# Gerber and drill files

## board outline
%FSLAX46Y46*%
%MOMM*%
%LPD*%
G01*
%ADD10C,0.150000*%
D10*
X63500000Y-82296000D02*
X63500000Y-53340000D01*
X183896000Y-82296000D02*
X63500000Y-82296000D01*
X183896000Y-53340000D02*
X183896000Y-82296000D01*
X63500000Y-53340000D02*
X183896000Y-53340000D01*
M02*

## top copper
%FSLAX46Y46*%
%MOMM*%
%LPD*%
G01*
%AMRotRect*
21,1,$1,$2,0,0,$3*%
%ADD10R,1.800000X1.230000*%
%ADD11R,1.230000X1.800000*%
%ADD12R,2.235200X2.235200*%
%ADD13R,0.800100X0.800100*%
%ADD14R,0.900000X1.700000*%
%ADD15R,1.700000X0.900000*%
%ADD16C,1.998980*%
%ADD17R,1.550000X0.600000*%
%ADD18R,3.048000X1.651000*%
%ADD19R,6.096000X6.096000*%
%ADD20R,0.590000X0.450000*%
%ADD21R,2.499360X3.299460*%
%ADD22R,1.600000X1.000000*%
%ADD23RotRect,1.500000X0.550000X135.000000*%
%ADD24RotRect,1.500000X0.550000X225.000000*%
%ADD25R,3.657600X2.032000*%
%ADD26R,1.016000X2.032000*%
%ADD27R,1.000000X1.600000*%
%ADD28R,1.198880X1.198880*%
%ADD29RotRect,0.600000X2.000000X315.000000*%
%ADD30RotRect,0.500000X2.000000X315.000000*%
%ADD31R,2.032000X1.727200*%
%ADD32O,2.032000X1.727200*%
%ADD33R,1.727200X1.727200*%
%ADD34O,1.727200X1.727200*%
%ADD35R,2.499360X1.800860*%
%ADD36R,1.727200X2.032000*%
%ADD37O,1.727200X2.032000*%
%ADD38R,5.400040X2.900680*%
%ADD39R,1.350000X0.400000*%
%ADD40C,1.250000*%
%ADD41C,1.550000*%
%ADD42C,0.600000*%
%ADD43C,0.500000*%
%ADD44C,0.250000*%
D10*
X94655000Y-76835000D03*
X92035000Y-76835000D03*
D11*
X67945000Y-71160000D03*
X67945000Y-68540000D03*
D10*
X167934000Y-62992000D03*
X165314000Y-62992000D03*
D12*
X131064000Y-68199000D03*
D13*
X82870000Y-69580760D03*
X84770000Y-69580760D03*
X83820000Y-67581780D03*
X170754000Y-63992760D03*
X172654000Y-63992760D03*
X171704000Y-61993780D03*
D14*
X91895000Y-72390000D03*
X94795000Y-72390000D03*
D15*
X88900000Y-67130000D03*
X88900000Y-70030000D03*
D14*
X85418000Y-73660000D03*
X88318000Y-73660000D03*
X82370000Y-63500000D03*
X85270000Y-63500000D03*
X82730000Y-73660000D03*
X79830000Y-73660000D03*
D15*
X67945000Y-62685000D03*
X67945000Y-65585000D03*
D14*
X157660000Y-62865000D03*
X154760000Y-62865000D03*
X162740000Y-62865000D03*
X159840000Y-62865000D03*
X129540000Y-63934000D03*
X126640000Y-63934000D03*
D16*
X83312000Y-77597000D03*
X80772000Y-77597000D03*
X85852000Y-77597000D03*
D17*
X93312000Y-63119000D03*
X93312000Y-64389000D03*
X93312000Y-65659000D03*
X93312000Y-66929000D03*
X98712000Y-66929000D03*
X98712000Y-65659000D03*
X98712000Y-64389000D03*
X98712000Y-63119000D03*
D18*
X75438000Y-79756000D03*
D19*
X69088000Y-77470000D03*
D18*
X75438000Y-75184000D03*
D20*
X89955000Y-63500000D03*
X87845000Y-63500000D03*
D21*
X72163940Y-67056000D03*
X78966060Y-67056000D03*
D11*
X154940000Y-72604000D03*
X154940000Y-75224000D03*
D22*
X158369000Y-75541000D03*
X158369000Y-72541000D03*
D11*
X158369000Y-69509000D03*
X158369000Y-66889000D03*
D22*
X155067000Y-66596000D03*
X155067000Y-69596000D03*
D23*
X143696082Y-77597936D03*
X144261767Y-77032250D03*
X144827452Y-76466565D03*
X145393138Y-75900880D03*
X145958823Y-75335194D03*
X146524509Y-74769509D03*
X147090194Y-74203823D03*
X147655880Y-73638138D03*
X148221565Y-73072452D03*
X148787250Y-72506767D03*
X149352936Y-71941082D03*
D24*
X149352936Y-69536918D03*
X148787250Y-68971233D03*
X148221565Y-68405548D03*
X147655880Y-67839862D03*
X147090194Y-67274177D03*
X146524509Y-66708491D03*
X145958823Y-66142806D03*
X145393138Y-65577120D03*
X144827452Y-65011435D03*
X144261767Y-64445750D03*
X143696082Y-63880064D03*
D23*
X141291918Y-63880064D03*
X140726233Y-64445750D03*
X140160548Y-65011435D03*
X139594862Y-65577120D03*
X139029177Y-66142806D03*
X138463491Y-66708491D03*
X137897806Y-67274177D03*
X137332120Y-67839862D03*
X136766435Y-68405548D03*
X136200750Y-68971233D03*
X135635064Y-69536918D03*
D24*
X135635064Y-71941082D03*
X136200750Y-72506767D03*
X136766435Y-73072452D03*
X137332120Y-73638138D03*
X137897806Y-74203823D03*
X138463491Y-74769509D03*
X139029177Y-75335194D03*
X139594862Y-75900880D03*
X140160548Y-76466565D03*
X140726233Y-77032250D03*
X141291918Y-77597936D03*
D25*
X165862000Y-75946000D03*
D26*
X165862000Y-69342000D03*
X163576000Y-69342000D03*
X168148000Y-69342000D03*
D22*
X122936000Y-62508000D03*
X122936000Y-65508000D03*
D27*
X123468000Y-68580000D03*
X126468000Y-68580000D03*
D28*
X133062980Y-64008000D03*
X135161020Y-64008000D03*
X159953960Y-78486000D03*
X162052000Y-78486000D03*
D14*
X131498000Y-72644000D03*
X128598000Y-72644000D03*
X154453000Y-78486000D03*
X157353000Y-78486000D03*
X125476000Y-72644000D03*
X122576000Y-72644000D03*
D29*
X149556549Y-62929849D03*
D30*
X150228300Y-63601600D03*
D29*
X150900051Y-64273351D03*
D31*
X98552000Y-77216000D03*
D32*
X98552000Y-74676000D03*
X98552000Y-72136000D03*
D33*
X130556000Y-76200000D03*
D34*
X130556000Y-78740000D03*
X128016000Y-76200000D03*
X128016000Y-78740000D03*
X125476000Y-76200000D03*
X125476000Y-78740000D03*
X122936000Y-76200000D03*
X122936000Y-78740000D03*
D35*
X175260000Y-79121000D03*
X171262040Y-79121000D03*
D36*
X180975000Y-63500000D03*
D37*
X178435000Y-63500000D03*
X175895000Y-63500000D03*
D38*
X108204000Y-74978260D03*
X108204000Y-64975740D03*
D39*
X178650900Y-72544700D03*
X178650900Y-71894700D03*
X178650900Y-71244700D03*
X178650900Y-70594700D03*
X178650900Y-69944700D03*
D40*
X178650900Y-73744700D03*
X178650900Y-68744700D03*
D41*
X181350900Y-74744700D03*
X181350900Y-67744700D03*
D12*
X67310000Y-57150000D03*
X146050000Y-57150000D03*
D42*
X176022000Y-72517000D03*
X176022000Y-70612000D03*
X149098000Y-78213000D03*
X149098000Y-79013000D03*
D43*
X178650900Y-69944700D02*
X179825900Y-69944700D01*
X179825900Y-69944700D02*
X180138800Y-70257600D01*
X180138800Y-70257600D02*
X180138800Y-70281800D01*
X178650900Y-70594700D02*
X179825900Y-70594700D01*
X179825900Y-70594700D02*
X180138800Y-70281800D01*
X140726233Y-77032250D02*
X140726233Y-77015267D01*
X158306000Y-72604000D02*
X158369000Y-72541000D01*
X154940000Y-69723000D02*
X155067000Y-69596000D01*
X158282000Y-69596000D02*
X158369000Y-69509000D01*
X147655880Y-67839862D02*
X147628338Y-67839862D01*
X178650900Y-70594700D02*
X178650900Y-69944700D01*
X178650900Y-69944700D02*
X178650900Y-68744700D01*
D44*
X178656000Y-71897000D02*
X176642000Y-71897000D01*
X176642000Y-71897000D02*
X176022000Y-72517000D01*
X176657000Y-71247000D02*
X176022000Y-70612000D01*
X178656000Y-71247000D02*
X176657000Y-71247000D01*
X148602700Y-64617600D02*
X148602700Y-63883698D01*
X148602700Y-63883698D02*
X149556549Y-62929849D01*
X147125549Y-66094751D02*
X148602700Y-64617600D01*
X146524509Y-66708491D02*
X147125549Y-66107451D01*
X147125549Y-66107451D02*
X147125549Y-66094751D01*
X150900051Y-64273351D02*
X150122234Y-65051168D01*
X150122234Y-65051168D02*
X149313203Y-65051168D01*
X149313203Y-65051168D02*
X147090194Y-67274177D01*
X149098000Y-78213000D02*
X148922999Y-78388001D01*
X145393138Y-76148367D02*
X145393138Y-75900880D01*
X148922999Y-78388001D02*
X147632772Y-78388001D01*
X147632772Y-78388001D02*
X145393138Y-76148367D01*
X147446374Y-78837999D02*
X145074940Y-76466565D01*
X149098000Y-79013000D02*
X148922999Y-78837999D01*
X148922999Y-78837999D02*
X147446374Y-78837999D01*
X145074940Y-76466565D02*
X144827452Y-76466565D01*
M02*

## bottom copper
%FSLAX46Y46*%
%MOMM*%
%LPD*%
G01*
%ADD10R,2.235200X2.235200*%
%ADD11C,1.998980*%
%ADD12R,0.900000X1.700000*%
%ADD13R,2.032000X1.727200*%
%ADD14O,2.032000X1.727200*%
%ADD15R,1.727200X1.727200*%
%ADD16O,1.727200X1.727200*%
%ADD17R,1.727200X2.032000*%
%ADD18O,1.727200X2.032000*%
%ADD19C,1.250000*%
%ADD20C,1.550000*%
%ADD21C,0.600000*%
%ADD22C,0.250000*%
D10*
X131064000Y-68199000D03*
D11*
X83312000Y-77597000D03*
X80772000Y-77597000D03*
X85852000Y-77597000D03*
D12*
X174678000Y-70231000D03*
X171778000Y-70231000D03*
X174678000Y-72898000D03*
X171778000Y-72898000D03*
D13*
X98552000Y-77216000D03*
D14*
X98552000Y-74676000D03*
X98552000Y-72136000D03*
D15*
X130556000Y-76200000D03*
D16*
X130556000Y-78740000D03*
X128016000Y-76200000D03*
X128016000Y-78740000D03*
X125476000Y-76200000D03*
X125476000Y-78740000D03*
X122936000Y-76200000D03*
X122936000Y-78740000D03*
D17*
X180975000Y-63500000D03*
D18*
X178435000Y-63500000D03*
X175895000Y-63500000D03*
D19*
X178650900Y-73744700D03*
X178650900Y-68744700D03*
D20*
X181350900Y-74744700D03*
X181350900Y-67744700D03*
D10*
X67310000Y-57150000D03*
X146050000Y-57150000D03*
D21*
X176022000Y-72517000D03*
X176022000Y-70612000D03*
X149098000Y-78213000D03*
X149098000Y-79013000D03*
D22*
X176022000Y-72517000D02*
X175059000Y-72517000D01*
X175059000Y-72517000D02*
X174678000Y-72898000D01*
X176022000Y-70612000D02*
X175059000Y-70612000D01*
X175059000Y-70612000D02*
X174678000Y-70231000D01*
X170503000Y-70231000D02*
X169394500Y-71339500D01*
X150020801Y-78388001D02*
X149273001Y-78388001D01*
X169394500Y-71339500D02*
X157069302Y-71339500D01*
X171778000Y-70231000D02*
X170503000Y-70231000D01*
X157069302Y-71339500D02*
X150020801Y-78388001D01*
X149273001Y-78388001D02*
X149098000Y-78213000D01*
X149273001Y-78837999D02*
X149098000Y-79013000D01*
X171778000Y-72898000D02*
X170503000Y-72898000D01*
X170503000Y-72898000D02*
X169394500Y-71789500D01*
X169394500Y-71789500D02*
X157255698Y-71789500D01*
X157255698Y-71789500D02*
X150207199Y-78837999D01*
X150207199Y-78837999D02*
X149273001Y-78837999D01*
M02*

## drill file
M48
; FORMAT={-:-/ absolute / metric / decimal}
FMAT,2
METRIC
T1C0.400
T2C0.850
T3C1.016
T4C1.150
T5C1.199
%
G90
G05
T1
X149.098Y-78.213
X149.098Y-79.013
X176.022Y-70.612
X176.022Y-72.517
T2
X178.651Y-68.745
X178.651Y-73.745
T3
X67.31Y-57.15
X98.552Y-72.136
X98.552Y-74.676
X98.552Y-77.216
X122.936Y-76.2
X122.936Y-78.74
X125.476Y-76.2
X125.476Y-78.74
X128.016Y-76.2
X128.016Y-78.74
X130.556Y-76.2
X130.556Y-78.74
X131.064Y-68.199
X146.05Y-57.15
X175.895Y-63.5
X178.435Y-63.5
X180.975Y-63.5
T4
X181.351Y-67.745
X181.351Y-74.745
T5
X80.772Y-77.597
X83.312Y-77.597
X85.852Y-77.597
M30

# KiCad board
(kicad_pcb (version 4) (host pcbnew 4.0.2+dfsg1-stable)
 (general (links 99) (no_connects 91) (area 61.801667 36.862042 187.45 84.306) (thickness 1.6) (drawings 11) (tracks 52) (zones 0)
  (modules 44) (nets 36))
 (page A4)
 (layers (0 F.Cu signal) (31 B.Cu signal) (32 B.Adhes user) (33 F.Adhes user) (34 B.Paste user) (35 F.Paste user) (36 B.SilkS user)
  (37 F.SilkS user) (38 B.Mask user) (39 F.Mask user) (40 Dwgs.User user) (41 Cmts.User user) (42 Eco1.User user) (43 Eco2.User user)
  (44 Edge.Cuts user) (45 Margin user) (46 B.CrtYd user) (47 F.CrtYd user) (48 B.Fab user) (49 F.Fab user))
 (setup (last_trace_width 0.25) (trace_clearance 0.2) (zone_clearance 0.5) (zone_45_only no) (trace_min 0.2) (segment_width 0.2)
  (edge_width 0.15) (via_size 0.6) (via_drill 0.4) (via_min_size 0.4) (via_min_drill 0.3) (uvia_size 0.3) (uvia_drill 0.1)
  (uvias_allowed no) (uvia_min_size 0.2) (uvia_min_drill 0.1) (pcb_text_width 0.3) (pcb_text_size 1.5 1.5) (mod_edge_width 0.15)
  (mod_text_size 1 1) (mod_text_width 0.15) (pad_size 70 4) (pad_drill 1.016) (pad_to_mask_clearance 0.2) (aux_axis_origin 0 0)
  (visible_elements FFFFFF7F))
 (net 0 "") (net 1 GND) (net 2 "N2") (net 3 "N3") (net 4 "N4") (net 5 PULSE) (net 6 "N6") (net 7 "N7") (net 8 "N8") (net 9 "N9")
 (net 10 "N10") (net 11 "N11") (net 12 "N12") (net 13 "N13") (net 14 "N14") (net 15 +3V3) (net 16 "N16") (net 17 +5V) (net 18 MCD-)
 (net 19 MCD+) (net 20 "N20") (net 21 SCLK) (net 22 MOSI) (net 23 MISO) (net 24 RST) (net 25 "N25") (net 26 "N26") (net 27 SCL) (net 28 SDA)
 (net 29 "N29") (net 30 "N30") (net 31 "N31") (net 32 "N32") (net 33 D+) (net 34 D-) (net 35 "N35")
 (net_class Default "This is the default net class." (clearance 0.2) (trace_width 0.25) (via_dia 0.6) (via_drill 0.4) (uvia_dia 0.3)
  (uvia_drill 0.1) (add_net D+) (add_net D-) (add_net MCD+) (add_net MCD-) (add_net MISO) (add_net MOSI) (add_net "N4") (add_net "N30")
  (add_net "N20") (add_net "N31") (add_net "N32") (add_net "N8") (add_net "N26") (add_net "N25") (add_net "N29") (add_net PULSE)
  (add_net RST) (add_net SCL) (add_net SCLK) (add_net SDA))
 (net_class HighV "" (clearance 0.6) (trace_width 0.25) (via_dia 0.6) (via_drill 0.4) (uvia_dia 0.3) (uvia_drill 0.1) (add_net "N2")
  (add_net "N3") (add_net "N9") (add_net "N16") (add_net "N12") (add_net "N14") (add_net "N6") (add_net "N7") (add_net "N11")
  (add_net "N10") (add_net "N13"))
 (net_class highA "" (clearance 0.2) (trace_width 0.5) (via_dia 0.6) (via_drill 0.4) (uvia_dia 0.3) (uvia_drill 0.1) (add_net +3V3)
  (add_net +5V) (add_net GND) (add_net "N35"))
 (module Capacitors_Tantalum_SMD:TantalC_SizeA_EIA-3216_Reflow (layer F.Cu) (at 93.345 76.835)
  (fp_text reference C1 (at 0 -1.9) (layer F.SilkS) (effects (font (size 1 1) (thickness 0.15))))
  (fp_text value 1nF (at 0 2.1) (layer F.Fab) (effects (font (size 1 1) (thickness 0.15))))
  (pad 2 smd rect (at 1.31 0) (size 1.8 1.23) (layers F.Cu F.Paste F.Mask) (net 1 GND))
  (pad 1 smd rect (at -1.31 0) (size 1.8 1.23) (layers F.Cu F.Paste F.Mask) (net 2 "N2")))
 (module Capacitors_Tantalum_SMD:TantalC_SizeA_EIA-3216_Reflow (layer F.Cu) (at 67.945 69.85 270)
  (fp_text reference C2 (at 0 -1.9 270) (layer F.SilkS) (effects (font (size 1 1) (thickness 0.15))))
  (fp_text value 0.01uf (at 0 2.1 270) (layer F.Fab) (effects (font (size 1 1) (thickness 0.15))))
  (pad 2 smd rect (at 1.31 0 270) (size 1.8 1.23) (layers F.Cu F.Paste F.Mask) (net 1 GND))
  (pad 1 smd rect (at -1.31 0 270) (size 1.8 1.23) (layers F.Cu F.Paste F.Mask) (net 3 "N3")))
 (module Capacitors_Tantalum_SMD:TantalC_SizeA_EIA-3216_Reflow (layer F.Cu) (at 166.624 62.992)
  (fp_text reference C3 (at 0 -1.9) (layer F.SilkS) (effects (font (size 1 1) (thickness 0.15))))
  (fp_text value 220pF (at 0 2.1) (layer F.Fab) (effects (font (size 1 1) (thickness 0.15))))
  (pad 2 smd rect (at 1.31 0) (size 1.8 1.23) (layers F.Cu F.Paste F.Mask) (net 1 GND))
  (pad 1 smd rect (at -1.31 0) (size 1.8 1.23) (layers F.Cu F.Paste F.Mask) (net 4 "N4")))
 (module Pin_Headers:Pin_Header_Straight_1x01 (layer F.Cu) (at 131.064 68.199)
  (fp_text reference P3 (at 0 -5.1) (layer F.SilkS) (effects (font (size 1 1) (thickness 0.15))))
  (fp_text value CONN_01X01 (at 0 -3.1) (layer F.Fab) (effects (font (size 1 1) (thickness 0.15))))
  (pad 1 thru_hole rect (at 0 0) (size 2.2352 2.2352) (drill 1.016) (layers *.Cu *.Mask F.SilkS) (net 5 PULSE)))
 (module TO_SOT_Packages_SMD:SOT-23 (layer F.Cu) (at 83.82 68.58)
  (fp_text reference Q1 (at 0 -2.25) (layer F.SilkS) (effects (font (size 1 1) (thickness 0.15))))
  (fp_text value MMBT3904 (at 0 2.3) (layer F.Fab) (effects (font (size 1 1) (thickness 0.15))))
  (pad 1 smd rect (at -0.95 1.00076) (size 0.8001 0.8001) (layers F.Cu F.Paste F.Mask) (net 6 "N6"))
  (pad 2 smd rect (at 0.95 1.00076) (size 0.8001 0.8001) (layers F.Cu F.Paste F.Mask) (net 1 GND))
  (pad 3 smd rect (at 0 -0.99822) (size 0.8001 0.8001) (layers F.Cu F.Paste F.Mask) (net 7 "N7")))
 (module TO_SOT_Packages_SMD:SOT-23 (layer F.Cu) (at 171.704 62.992)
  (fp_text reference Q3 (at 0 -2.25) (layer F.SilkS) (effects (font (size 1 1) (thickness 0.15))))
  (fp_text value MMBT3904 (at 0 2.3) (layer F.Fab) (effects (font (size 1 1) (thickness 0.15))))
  (pad 1 smd rect (at -0.95 1.00076) (size 0.8001 0.8001) (layers F.Cu F.Paste F.Mask) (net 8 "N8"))
  (pad 2 smd rect (at 0.95 1.00076) (size 0.8001 0.8001) (layers F.Cu F.Paste F.Mask) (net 1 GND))
  (pad 3 smd rect (at 0 -0.99822) (size 0.8001 0.8001) (layers F.Cu F.Paste F.Mask) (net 5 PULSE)))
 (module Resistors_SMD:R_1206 (layer F.Cu) (at 93.345 72.39)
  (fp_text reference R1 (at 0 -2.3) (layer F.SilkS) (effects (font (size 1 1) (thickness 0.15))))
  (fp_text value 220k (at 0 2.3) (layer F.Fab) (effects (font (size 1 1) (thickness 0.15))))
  (pad 1 smd rect (at -1.45 0) (size 0.9 1.7) (layers F.Cu F.Paste F.Mask) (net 2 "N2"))
  (pad 2 smd rect (at 1.45 0) (size 0.9 1.7) (layers F.Cu F.Paste F.Mask) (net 1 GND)))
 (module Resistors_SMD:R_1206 (layer F.Cu) (at 88.9 68.58 270)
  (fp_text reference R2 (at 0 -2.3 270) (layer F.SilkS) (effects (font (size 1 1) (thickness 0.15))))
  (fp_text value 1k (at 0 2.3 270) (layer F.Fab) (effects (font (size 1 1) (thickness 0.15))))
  (pad 1 smd rect (at -1.45 0 270) (size 0.9 1.7) (layers F.Cu F.Paste F.Mask) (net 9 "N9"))
  (pad 2 smd rect (at 1.45 0 270) (size 0.9 1.7) (layers F.Cu F.Paste F.Mask) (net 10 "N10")))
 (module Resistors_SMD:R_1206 (layer F.Cu) (at 86.868 73.66)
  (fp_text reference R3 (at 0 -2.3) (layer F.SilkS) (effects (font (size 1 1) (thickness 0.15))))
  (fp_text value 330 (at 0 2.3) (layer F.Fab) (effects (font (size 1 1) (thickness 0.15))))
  (pad 1 smd rect (at -1.45 0) (size 0.9 1.7) (layers F.Cu F.Paste F.Mask) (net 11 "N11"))
  (pad 2 smd rect (at 1.45 0) (size 0.9 1.7) (layers F.Cu F.Paste F.Mask) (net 10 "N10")))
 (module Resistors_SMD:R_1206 (layer F.Cu) (at 83.82 63.5)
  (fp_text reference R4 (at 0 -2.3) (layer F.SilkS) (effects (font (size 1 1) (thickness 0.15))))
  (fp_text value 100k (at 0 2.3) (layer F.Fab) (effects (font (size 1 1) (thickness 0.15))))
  (pad 1 smd rect (at -1.45 0) (size 0.9 1.7) (layers F.Cu F.Paste F.Mask) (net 7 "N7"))
  (pad 2 smd rect (at 1.45 0) (size 0.9 1.7) (layers F.Cu F.Paste F.Mask) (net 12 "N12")))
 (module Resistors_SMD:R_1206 (layer F.Cu) (at 81.28 73.66 180)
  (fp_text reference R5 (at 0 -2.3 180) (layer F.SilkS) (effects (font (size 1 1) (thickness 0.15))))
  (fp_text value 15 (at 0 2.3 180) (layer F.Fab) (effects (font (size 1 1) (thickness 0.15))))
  (pad 1 smd rect (at -1.45 0 180) (size 0.9 1.7) (layers F.Cu F.Paste F.Mask) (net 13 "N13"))
  (pad 2 smd rect (at 1.45 0 180) (size 0.9 1.7) (layers F.Cu F.Paste F.Mask) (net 6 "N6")))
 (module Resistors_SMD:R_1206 (layer F.Cu) (at 67.945 64.135 270)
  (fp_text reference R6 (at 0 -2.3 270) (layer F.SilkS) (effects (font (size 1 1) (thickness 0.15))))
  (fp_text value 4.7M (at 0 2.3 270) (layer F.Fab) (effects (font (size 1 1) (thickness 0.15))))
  (pad 1 smd rect (at -1.45 0 270) (size 0.9 1.7) (layers F.Cu F.Paste F.Mask) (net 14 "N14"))
  (pad 2 smd rect (at 1.45 0 270) (size 0.9 1.7) (layers F.Cu F.Paste F.Mask) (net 3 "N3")))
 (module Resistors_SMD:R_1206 (layer F.Cu) (at 156.21 62.865 180)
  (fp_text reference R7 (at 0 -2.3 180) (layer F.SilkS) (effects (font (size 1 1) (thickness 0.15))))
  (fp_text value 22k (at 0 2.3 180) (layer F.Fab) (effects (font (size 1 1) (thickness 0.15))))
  (pad 1 smd rect (at -1.45 0 180) (size 0.9 1.7) (layers F.Cu F.Paste F.Mask) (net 8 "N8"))
  (pad 2 smd rect (at 1.45 0 180) (size 0.9 1.7) (layers F.Cu F.Paste F.Mask) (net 4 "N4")))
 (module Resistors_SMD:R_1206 (layer F.Cu) (at 161.29 62.865 180)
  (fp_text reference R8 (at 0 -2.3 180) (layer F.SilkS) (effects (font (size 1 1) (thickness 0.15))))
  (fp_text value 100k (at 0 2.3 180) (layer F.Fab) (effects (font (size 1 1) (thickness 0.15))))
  (pad 1 smd rect (at -1.45 0 180) (size 0.9 1.7) (layers F.Cu F.Paste F.Mask) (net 1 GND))
  (pad 2 smd rect (at 1.45 0 180) (size 0.9 1.7) (layers F.Cu F.Paste F.Mask) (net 8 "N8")))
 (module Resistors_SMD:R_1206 (layer F.Cu) (at 128.09 63.934 180)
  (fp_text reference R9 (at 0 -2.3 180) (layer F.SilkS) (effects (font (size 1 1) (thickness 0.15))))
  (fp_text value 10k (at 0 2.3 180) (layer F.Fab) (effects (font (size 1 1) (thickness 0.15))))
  (pad 1 smd rect (at -1.45 0 180) (size 0.9 1.7) (layers F.Cu F.Paste F.Mask) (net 5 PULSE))
  (pad 2 smd rect (at 1.45 0 180) (size 0.9 1.7) (layers F.Cu F.Paste F.Mask) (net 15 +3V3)))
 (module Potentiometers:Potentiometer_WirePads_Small (layer F.Cu) (at 85.852 77.597 270)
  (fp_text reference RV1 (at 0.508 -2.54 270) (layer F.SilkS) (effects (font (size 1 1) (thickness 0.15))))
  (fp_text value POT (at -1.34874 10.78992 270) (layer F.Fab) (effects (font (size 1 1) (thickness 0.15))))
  (pad 2 thru_hole circle (at 0 2.54 270) (size 1.99898 1.99898) (drill 1.19888) (layers *.Cu *.Mask F.SilkS) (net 13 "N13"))
  (pad 3 thru_hole circle (at 0 5.08 270) (size 1.99898 1.99898) (drill 1.19888) (layers *.Cu *.Mask F.SilkS) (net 1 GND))
  (pad 1 thru_hole circle (at 0 0 270) (size 1.99898 1.99898) (drill 1.19888) (layers *.Cu *.Mask F.SilkS) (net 13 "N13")))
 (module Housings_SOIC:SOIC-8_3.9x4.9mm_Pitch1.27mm (layer F.Cu) (at 96.012 65.024)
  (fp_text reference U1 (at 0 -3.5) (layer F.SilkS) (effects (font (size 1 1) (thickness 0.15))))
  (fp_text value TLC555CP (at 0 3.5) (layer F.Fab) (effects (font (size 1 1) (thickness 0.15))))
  (pad 1 smd rect (at -2.7 -1.905) (size 1.55 0.6) (layers F.Cu F.Paste F.Mask) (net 1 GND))
  (pad 2 smd rect (at -2.7 -0.635) (size 1.55 0.6) (layers F.Cu F.Paste F.Mask) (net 2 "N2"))
  (pad 3 smd rect (at -2.7 0.635) (size 1.55 0.6) (layers F.Cu F.Paste F.Mask) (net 10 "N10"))
  (pad 4 smd rect (at -2.7 1.905) (size 1.55 0.6) (layers F.Cu F.Paste F.Mask) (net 7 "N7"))
  (pad 5 smd rect (at 2.7 1.905) (size 1.55 0.6) (layers F.Cu F.Paste F.Mask))
  (pad 6 smd rect (at 2.7 0.635) (size 1.55 0.6) (layers F.Cu F.Paste F.Mask) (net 1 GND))
  (pad 7 smd rect (at 2.7 -0.635) (size 1.55 0.6) (layers F.Cu F.Paste F.Mask) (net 11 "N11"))
  (pad 8 smd rect (at 2.7 -1.905) (size 1.55 0.6) (layers F.Cu F.Paste F.Mask) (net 12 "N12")))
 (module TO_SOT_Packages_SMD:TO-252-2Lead (layer F.Cu) (at 75.438 77.47 90)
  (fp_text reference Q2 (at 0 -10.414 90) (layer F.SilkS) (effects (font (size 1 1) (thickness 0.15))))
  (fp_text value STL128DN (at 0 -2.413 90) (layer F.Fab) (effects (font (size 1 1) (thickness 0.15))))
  (pad 1 smd rect (at -2.286 0 90) (size 1.651 3.048) (layers F.Cu F.Paste F.Mask) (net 11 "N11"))
  (pad 2 smd rect (at 0 -6.35 90) (size 6.096 6.096) (layers F.Cu F.Paste F.Mask) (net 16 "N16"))
  (pad 3 smd rect (at 2.286 0 90) (size 1.651 3.048) (layers F.Cu F.Paste F.Mask) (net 6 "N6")))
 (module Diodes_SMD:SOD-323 (layer F.Cu) (at 88.9 63.5 180)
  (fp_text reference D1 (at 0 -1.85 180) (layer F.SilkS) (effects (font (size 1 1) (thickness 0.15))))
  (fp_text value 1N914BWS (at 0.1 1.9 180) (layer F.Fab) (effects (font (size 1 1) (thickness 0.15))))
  (pad 1 smd rect (at -1.055 0 180) (size 0.59 0.45) (layers F.Cu F.Paste F.Mask) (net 2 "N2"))
  (pad 2 smd rect (at 1.055 0 180) (size 0.59 0.45) (layers F.Cu F.Paste F.Mask) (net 9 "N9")))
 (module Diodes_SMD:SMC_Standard (layer F.Cu) (at 75.565 67.056)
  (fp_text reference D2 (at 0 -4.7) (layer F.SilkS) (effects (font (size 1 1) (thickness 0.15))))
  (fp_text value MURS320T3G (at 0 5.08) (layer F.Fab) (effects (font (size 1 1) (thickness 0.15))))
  (pad 1 smd rect (at -3.40106 0 90) (size 3.29946 2.49936) (layers F.Cu F.Paste F.Mask) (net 3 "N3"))
  (pad 2 smd rect (at 3.40106 0 90) (size 3.29946 2.49936) (layers F.Cu F.Paste F.Mask) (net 16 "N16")))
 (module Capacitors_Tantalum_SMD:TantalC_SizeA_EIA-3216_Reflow (layer F.Cu) (at 154.94 73.914 90)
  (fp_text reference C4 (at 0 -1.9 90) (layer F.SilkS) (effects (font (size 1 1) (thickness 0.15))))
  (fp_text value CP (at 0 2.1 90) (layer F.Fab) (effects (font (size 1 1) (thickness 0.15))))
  (pad 2 smd rect (at 1.31 0 90) (size 1.8 1.23) (layers F.Cu F.Paste F.Mask) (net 1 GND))
  (pad 1 smd rect (at -1.31 0 90) (size 1.8 1.23) (layers F.Cu F.Paste F.Mask) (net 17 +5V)))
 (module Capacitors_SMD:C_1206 (layer F.Cu) (at 158.369 74.041 90)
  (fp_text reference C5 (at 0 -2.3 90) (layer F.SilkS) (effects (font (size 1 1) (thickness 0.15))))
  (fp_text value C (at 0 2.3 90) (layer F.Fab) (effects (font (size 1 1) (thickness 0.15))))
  (pad 1 smd rect (at -1.5 0 90) (size 1 1.6) (layers F.Cu F.Paste F.Mask) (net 17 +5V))
  (pad 2 smd rect (at 1.5 0 90) (size 1 1.6) (layers F.Cu F.Paste F.Mask) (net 1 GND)))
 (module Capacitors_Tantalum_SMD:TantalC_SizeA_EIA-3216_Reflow (layer F.Cu) (at 158.369 68.199 270)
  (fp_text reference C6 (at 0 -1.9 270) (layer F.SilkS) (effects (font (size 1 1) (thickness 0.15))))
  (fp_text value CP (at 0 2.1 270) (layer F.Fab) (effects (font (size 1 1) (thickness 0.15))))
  (pad 2 smd rect (at 1.31 0 270) (size 1.8 1.23) (layers F.Cu F.Paste F.Mask) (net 1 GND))
  (pad 1 smd rect (at -1.31 0 270) (size 1.8 1.23) (layers F.Cu F.Paste F.Mask) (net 15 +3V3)))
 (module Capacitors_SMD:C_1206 (layer F.Cu) (at 155.067 68.096 270)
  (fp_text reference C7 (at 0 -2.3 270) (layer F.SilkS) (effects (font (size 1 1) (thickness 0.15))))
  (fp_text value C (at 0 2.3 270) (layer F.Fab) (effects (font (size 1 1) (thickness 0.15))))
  (pad 1 smd rect (at -1.5 0 270) (size 1 1.6) (layers F.Cu F.Paste F.Mask) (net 15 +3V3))
  (pad 2 smd rect (at 1.5 0 270) (size 1 1.6) (layers F.Cu F.Paste F.Mask) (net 1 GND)))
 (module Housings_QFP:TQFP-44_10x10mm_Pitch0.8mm (layer F.Cu) (at 142.494 70.739 135)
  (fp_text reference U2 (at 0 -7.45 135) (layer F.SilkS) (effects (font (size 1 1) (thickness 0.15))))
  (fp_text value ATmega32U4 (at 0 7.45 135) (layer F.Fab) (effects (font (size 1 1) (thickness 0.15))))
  (pad 1 smd rect (at -5.7 -4 135) (size 1.5 0.55) (layers F.Cu F.Paste F.Mask))
  (pad 2 smd rect (at -5.7 -3.2 135) (size 1.5 0.55) (layers F.Cu F.Paste F.Mask) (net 17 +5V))
  (pad 3 smd rect (at -5.7 -2.4 135) (size 1.5 0.55) (layers F.Cu F.Paste F.Mask) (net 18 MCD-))
  (pad 4 smd rect (at -5.7 -1.6 135) (size 1.5 0.55) (layers F.Cu F.Paste F.Mask) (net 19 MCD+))
  (pad 5 smd rect (at -5.7 -0.8 135) (size 1.5 0.55) (layers F.Cu F.Paste F.Mask) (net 1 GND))
  (pad 6 smd rect (at -5.7 0 135) (size 1.5 0.55) (layers F.Cu F.Paste F.Mask) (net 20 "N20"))
  (pad 7 smd rect (at -5.7 0.8 135) (size 1.5 0.55) (layers F.Cu F.Paste F.Mask) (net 17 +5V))
  (pad 8 smd rect (at -5.7 1.6 135) (size 1.5 0.55) (layers F.Cu F.Paste F.Mask))
  (pad 9 smd rect (at -5.7 2.4 135) (size 1.5 0.55) (layers F.Cu F.Paste F.Mask) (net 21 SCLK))
  (pad 10 smd rect (at -5.7 3.2 135) (size 1.5 0.55) (layers F.Cu F.Paste F.Mask) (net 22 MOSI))
  (pad 11 smd rect (at -5.7 4 135) (size 1.5 0.55) (layers F.Cu F.Paste F.Mask) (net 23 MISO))
  (pad 12 smd rect (at -4 5.7 225) (size 1.5 0.55) (layers F.Cu F.Paste F.Mask))
  (pad 13 smd rect (at -3.2 5.7 225) (size 1.5 0.55) (layers F.Cu F.Paste F.Mask) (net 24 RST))
  (pad 14 smd rect (at -2.4 5.7 225) (size 1.5 0.55) (layers F.Cu F.Paste F.Mask) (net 17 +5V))
  (pad 15 smd rect (at -1.6 5.7 225) (size 1.5 0.55) (layers F.Cu F.Paste F.Mask) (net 1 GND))
  (pad 16 smd rect (at -0.8 5.7 225) (size 1.5 0.55) (layers F.Cu F.Paste F.Mask) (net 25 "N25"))
  (pad 17 smd rect (at 0 5.7 225) (size 1.5 0.55) (layers F.Cu F.Paste F.Mask) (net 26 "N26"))
  (pad 18 smd rect (at 0.8 5.7 225) (size 1.5 0.55) (layers F.Cu F.Paste F.Mask) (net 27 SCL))
  (pad 19 smd rect (at 1.6 5.7 225) (size 1.5 0.55) (layers F.Cu F.Paste F.Mask) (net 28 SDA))
  (pad 20 smd rect (at 2.4 5.7 225) (size 1.5 0.55) (layers F.Cu F.Paste F.Mask))
  (pad 21 smd rect (at 3.2 5.7 225) (size 1.5 0.55) (layers F.Cu F.Paste F.Mask))
  (pad 22 smd rect (at 4 5.7 225) (size 1.5 0.55) (layers F.Cu F.Paste F.Mask))
  (pad 23 smd rect (at 5.7 4 135) (size 1.5 0.55) (layers F.Cu F.Paste F.Mask) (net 1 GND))
  (pad 24 smd rect (at 5.7 3.2 135) (size 1.5 0.55) (layers F.Cu F.Paste F.Mask) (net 17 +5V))
  (pad 25 smd rect (at 5.7 2.4 135) (size 1.5 0.55) (layers F.Cu F.Paste F.Mask))
  (pad 26 smd rect (at 5.7 1.6 135) (size 1.5 0.55) (layers F.Cu F.Paste F.Mask))
  (pad 27 smd rect (at 5.7 0.8 135) (size 1.5 0.55) (layers F.Cu F.Paste F.Mask))
  (pad 28 smd rect (at 5.7 0 135) (size 1.5 0.55) (layers F.Cu F.Paste F.Mask))
  (pad 29 smd rect (at 5.7 -0.8 135) (size 1.5 0.55) (layers F.Cu F.Paste F.Mask))
  (pad 30 smd rect (at 5.7 -1.6 135) (size 1.5 0.55) (layers F.Cu F.Paste F.Mask) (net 5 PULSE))
  (pad 31 smd rect (at 5.7 -2.4 135) (size 1.5 0.55) (layers F.Cu F.Paste F.Mask))
  (pad 32 smd rect (at 5.7 -3.2 135) (size 1.5 0.55) (layers F.Cu F.Paste F.Mask))
  (pad 33 smd rect (at 5.7 -4 135) (size 1.5 0.55) (layers F.Cu F.Paste F.Mask))
  (pad 34 smd rect (at 4 -5.7 225) (size 1.5 0.55) (layers F.Cu F.Paste F.Mask) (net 17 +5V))
  (pad 35 smd rect (at 3.2 -5.7 225) (size 1.5 0.55) (layers F.Cu F.Paste F.Mask) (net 1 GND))
  (pad 36 smd rect (at 2.4 -5.7 225) (size 1.5 0.55) (layers F.Cu F.Paste F.Mask) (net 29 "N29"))
  (pad 37 smd rect (at 1.6 -5.7 225) (size 1.5 0.55) (layers F.Cu F.Paste F.Mask))
  (pad 38 smd rect (at 0.8 -5.7 225) (size 1.5 0.55) (layers F.Cu F.Paste F.Mask))
  (pad 39 smd rect (at 0 -5.7 225) (size 1.5 0.55) (layers F.Cu F.Paste F.Mask))
  (pad 40 smd rect (at -0.8 -5.7 225) (size 1.5 0.55) (layers F.Cu F.Paste F.Mask))
  (pad 41 smd rect (at -1.6 -5.7 225) (size 1.5 0.55) (layers F.Cu F.Paste F.Mask))
  (pad 42 smd rect (at -2.4 -5.7 225) (size 1.5 0.55) (layers F.Cu F.Paste F.Mask) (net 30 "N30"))
  (pad 43 smd rect (at -3.2 -5.7 225) (size 1.5 0.55) (layers F.Cu F.Paste F.Mask) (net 1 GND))
  (pad 44 smd rect (at -4 -5.7 225) (size 1.5 0.55) (layers F.Cu F.Paste F.Mask) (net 17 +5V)))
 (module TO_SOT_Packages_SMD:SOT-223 (layer F.Cu) (at 165.862 72.644 180)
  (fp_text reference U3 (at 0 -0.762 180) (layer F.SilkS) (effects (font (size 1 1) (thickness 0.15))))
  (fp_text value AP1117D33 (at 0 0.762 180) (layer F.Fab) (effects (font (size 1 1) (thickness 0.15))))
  (pad 4 smd rect (at 0 -3.302 180) (size 3.6576 2.032) (layers F.Cu F.Paste F.Mask))
  (pad 2 smd rect (at 0 3.302 180) (size 1.016 2.032) (layers F.Cu F.Paste F.Mask) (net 15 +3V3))
  (pad 3 smd rect (at 2.286 3.302 180) (size 1.016 2.032) (layers F.Cu F.Paste F.Mask) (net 17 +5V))
  (pad 1 smd rect (at -2.286 3.302 180) (size 1.016 2.032) (layers F.Cu F.Paste F.Mask) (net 1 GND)))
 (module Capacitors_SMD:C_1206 (layer F.Cu) (at 122.936 64.008 270)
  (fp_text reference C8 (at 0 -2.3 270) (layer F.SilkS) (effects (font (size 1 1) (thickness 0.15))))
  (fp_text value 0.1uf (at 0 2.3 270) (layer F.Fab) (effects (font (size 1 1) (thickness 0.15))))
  (pad 1 smd rect (at -1.5 0 270) (size 1 1.6) (layers F.Cu F.Paste F.Mask) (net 30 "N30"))
  (pad 2 smd rect (at 1.5 0 270) (size 1 1.6) (layers F.Cu F.Paste F.Mask) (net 1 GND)))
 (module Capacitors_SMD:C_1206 (layer F.Cu) (at 124.968 68.58)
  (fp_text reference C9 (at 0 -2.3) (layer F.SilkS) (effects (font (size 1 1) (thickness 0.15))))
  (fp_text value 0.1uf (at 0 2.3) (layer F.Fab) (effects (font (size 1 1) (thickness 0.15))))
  (pad 1 smd rect (at -1.5 0) (size 1 1.6) (layers F.Cu F.Paste F.Mask) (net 1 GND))
  (pad 2 smd rect (at 1.5 0) (size 1 1.6) (layers F.Cu F.Paste F.Mask) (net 20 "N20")))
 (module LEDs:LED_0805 (layer F.Cu) (at 134.112 64.008 180)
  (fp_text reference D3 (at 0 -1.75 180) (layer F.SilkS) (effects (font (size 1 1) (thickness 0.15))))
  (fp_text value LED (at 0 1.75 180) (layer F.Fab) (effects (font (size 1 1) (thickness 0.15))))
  (pad 2 smd rect (at 1.04902 0) (size 1.19888 1.19888) (layers F.Cu F.Paste F.Mask) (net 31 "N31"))
  (pad 1 smd rect (at -1.04902 0) (size 1.19888 1.19888) (layers F.Cu F.Paste F.Mask) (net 1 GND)))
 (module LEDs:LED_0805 (layer F.Cu) (at 161.00298 78.486 180)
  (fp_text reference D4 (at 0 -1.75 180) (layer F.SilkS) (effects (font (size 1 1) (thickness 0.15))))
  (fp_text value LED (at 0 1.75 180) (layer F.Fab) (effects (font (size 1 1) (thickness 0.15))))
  (pad 2 smd rect (at 1.04902 0) (size 1.19888 1.19888) (layers F.Cu F.Paste F.Mask) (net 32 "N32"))
  (pad 1 smd rect (at -1.04902 0) (size 1.19888 1.19888) (layers F.Cu F.Paste F.Mask) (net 1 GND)))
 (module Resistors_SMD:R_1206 (layer B.Cu) (at 173.228 70.231 180)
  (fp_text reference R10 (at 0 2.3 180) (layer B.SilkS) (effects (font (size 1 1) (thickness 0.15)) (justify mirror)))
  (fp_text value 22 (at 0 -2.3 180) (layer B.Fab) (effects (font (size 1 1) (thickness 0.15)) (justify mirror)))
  (pad 1 smd rect (at -1.45 0 180) (size 0.9 1.7) (layers B.Cu B.Paste B.Mask) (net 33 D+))
  (pad 2 smd rect (at 1.45 0 180) (size 0.9 1.7) (layers B.Cu B.Paste B.Mask) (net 19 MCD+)))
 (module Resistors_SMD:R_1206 (layer B.Cu) (at 173.228 72.898 180)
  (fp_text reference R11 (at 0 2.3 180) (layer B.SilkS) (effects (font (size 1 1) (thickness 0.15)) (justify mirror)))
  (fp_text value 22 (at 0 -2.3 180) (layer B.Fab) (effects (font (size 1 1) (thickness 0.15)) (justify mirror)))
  (pad 1 smd rect (at -1.45 0 180) (size 0.9 1.7) (layers B.Cu B.Paste B.Mask) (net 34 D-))
  (pad 2 smd rect (at 1.45 0 180) (size 0.9 1.7) (layers B.Cu B.Paste B.Mask) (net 18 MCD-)))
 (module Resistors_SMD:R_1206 (layer F.Cu) (at 130.048 72.644 180)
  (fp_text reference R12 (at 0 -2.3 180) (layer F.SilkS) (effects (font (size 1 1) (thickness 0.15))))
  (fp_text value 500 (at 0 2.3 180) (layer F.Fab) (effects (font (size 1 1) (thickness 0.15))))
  (pad 1 smd rect (at -1.45 0 180) (size 0.9 1.7) (layers F.Cu F.Paste F.Mask) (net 31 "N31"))
  (pad 2 smd rect (at 1.45 0 180) (size 0.9 1.7) (layers F.Cu F.Paste F.Mask) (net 17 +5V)))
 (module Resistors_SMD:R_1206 (layer F.Cu) (at 155.903 78.486)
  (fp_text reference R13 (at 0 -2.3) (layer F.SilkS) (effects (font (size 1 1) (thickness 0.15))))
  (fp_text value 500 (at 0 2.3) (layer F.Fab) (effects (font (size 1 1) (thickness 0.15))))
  (pad 1 smd rect (at -1.45 0) (size 0.9 1.7) (layers F.Cu F.Paste F.Mask) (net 29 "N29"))
  (pad 2 smd rect (at 1.45 0) (size 0.9 1.7) (layers F.Cu F.Paste F.Mask) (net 32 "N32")))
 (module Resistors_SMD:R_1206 (layer F.Cu) (at 124.026 72.644 180)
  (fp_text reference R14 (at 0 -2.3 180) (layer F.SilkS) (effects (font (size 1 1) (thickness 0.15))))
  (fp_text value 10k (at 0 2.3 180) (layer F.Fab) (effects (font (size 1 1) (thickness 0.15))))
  (pad 1 smd rect (at -1.45 0 180) (size 0.9 1.7) (layers F.Cu F.Paste F.Mask) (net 17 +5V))
  (pad 2 smd rect (at 1.45 0 180) (size 0.9 1.7) (layers F.Cu F.Paste F.Mask) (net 24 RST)))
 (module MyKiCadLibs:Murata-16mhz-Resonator (layer F.Cu) (at 150.2283 63.6016 315)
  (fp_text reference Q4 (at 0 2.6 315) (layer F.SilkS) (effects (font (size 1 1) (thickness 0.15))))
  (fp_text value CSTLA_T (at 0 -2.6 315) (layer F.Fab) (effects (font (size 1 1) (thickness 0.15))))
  (pad 1 smd rect (at -0.95 0 315) (size 0.6 2) (layers F.Cu F.Paste F.Mask) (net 26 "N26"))
  (pad 2 smd rect (at 0 0 315) (size 0.5 2) (layers F.Cu F.Paste F.Mask) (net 1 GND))
  (pad 3 smd rect (at 0.95 0 315) (size 0.6 2) (layers F.Cu F.Paste F.Mask) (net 25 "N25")))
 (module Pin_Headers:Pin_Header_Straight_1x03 (layer F.Cu) (at 98.552 77.216 180)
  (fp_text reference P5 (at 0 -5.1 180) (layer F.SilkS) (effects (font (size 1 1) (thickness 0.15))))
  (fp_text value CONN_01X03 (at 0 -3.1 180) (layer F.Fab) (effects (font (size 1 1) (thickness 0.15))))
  (pad 1 thru_hole rect (at 0 0 180) (size 2.032 1.7272) (drill 1.016) (layers *.Cu *.Mask F.SilkS) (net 15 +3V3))
  (pad 2 thru_hole oval (at 0 2.54 180) (size 2.032 1.7272) (drill 1.016) (layers *.Cu *.Mask F.SilkS) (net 12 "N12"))
  (pad 3 thru_hole oval (at 0 5.08 180) (size 2.032 1.7272) (drill 1.016) (layers *.Cu *.Mask F.SilkS) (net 17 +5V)))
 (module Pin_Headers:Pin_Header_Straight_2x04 (layer F.Cu) (at 130.556 76.2 270)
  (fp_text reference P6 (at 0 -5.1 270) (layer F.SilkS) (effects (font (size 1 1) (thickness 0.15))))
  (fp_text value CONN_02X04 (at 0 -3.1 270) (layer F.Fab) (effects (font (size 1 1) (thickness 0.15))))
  (pad 1 thru_hole rect (at 0 0 270) (size 1.7272 1.7272) (drill 1.016) (layers *.Cu *.Mask F.SilkS) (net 23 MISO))
  (pad 2 thru_hole oval (at 2.54 0 270) (size 1.7272 1.7272) (drill 1.016) (layers *.Cu *.Mask F.SilkS) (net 17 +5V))
  (pad 3 thru_hole oval (at 0 2.54 270) (size 1.7272 1.7272) (drill 1.016) (layers *.Cu *.Mask F.SilkS) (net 21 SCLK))
  (pad 4 thru_hole oval (at 2.54 2.54 270) (size 1.7272 1.7272) (drill 1.016) (layers *.Cu *.Mask F.SilkS) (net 22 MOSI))
  (pad 5 thru_hole oval (at 0 5.08 270) (size 1.7272 1.7272) (drill 1.016) (layers *.Cu *.Mask F.SilkS) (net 24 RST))
  (pad 6 thru_hole oval (at 2.54 5.08 270) (size 1.7272 1.7272) (drill 1.016) (layers *.Cu *.Mask F.SilkS) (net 1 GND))
  (pad 7 thru_hole oval (at 0 7.62 270) (size 1.7272 1.7272) (drill 1.016) (layers *.Cu *.Mask F.SilkS) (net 27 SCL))
  (pad 8 thru_hole oval (at 2.54 7.62 270) (size 1.7272 1.7272) (drill 1.016) (layers *.Cu *.Mask F.SilkS) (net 28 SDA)))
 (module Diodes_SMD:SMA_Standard (layer F.Cu) (at 173.26102 79.121 180)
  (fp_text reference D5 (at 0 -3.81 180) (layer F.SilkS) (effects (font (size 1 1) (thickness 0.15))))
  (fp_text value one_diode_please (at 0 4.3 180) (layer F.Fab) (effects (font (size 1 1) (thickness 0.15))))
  (pad 1 smd rect (at -1.99898 0 180) (size 2.49936 1.80086) (layers F.Cu F.Paste F.Mask) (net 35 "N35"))
  (pad 2 smd rect (at 1.99898 0 180) (size 2.49936 1.80086) (layers F.Cu F.Paste F.Mask) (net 17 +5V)))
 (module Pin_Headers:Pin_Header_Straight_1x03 (layer F.Cu) (at 180.975 63.5 270)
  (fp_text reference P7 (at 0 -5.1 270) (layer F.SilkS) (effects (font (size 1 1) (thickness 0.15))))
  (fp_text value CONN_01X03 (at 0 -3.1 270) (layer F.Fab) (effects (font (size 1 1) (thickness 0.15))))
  (pad 1 thru_hole rect (at 0 0 270) (size 2.032 1.7272) (drill 1.016) (layers *.Cu *.Mask F.SilkS) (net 15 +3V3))
  (pad 2 thru_hole oval (at 0 2.54 270) (size 2.032 1.7272) (drill 1.016) (layers *.Cu *.Mask F.SilkS) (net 1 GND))
  (pad 3 thru_hole oval (at 0 5.08 270) (size 2.032 1.7272) (drill 1.016) (layers *.Cu *.Mask F.SilkS) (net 17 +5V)))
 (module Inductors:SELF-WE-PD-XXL (layer F.Cu) (at 108.204 69.977 90)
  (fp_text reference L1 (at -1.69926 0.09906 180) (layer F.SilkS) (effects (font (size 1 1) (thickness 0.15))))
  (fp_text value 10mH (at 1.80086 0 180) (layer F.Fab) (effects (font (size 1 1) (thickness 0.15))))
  (pad 1 smd rect (at -5.00126 0 90) (size 2.90068 5.40004) (layers F.Cu F.Paste F.Mask) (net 16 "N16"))
  (pad 2 smd rect (at 5.00126 0 90) (size 2.90068 5.40004) (layers F.Cu F.Paste F.Mask) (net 12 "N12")))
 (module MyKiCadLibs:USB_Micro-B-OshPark (layer F.Cu) (at 180.21344 71.2438 90)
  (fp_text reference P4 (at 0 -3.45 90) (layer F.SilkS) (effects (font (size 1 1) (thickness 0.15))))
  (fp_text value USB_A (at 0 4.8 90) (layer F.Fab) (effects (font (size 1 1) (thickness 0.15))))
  (pad 1 smd rect (at -1.3009 -1.56254 180) (size 1.35 0.4) (layers F.Cu F.Paste F.Mask) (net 35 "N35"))
  (pad 2 smd rect (at -0.6509 -1.56254 180) (size 1.35 0.4) (layers F.Cu F.Paste F.Mask) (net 34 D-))
  (pad 3 smd rect (at -0.0009 -1.56254 180) (size 1.35 0.4) (layers F.Cu F.Paste F.Mask) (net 33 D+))
  (pad 4 smd rect (at 0.6491 -1.56254 180) (size 1.35 0.4) (layers F.Cu F.Paste F.Mask) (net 1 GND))
  (pad 5 smd rect (at 1.2991 -1.56254 180) (size 1.35 0.4) (layers F.Cu F.Paste F.Mask) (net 1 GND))
  (pad 5 thru_hole circle (at -2.5009 -1.56254 270) (size 1.25 1.25) (drill 0.85) (layers *.Cu *.Mask F.SilkS) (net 1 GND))
  (pad 5 thru_hole circle (at 2.4991 -1.56254 180) (size 1.25 1.25) (drill 0.85) (layers *.Cu *.Mask F.SilkS) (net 1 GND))
  (pad 5 thru_hole circle (at -3.5009 1.13746 180) (size 1.55 1.55) (drill 1.15) (layers *.Cu *.Mask F.SilkS) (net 1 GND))
  (pad 5 thru_hole circle (at 3.4991 1.13746 180) (size 1.55 1.55) (drill 1.15) (layers *.Cu *.Mask F.SilkS) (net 1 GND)))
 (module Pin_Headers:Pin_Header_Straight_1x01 (layer F.Cu) (at 67.31 57.15)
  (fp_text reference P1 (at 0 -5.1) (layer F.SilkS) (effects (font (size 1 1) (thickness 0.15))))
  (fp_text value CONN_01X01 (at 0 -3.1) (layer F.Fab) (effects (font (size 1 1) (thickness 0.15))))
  (pad 1 thru_hole rect (at 0 0) (size 2.2352 2.2352) (drill 1.016) (layers *.Cu *.Mask F.SilkS) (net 14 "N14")))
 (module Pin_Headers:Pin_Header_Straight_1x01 (layer F.Cu) (at 146.05 57.15)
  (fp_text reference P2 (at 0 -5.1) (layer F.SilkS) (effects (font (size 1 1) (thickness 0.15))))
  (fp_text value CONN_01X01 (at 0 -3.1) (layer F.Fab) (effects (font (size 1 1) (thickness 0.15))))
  (pad 1 thru_hole rect (at 0 0) (size 2.2352 2.2352) (drill 1.016) (layers *.Cu *.Mask F.SilkS) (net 4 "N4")))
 (gr_line (start 63.5 82.296) (end 63.5 53.34) (layer Edge.Cuts) (width 0.15))
 (gr_line (start 183.896 82.296) (end 63.5 82.296) (layer Edge.Cuts) (width 0.15))
 (gr_line (start 183.896 53.34) (end 183.896 82.296) (layer Edge.Cuts) (width 0.15))
 (gr_line (start 63.5 53.34) (end 183.896 53.34) (layer Edge.Cuts) (width 0.15))
 (segment (start 178.6509 69.9447) (end 179.8259 69.9447) (width 0.5) (layer F.Cu) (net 1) (status 10))
 (segment (start 179.8259 69.9447) (end 180.1388 70.2576) (width 0.5) (layer F.Cu) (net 1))
 (segment (start 180.1388 70.2576) (end 180.1388 70.2818) (width 0.5) (layer F.Cu) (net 1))
 (segment (start 178.6509 70.5947) (end 179.8259 70.5947) (width 0.5) (layer F.Cu) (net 1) (status 10))
 (segment (start 179.8259 70.5947) (end 180.1388 70.2818) (width 0.5) (layer F.Cu) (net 1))
 (segment (start 140.726233 77.03225) (end 140.726233 77.015267) (width 0.5) (layer F.Cu) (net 1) (status 30))
 (segment (start 158.306 72.604) (end 158.369 72.541) (width 0.5) (layer F.Cu) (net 1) (status 30))
 (segment (start 154.94 69.723) (end 155.067 69.596) (width 0.5) (layer F.Cu) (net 1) (status 30))
 (segment (start 158.282 69.596) (end 158.369 69.509) (width 0.5) (layer F.Cu) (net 1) (status 30))
 (segment (start 147.65588 67.839862) (end 147.628338 67.839862) (width 0.5) (layer F.Cu) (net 1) (status 30))
 (segment (start 178.6509 70.5947) (end 178.6509 69.9447) (width 0.5) (layer F.Cu) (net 1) (status 30))
 (segment (start 178.6509 69.9447) (end 178.6509 68.7447) (width 0.5) (layer F.Cu) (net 1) (status 30))
 (segment (start 176.022 72.517) (end 175.059 72.517) (width 0.25) (layer B.Cu) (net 34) (status 20))
 (segment (start 175.059 72.517) (end 174.678 72.898) (width 0.25) (layer B.Cu) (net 34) (status 30))
 (segment (start 178.656 71.897) (end 176.642 71.897) (width 0.25) (layer F.Cu) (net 34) (status 10))
 (segment (start 176.642 71.897) (end 176.022 72.517) (width 0.25) (layer F.Cu) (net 34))
 (via (at 176.022 72.517) (size 0.6) (drill 0.4) (layers F.Cu B.Cu) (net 34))
 (segment (start 176.022 70.612) (end 175.059 70.612) (width 0.25) (layer B.Cu) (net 33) (status 20))
 (segment (start 175.059 70.612) (end 174.678 70.231) (width 0.25) (layer B.Cu) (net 33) (status 30))
 (segment (start 176.657 71.247) (end 176.022 70.612) (width 0.25) (layer F.Cu) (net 33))
 (via (at 176.022 70.612) (size 0.6) (drill 0.4) (layers F.Cu B.Cu) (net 33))
 (segment (start 178.656 71.247) (end 176.657 71.247) (width 0.25) (layer F.Cu) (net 33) (status 10))
 (segment (start 148.6027 64.6176) (end 148.6027 63.883698) (width 0.25) (layer F.Cu) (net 26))
 (segment (start 148.6027 63.883698) (end 149.556549 62.929849) (width 0.25) (layer F.Cu) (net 26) (status 20))
 (segment (start 147.125549 66.094751) (end 148.6027 64.6176) (width 0.25) (layer F.Cu) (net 26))
 (segment (start 146.524509 66.708491) (end 147.125549 66.107451) (width 0.25) (layer F.Cu) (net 26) (status 10))
 (segment (start 147.125549 66.107451) (end 147.125549 66.094751) (width 0.25) (layer F.Cu) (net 26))
 (segment (start 150.900051 64.273351) (end 150.122234 65.051168) (width 0.25) (layer F.Cu) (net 25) (status 10))
 (segment (start 150.122234 65.051168) (end 149.313203 65.051168) (width 0.25) (layer F.Cu) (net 25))
 (segment (start 149.313203 65.051168) (end 147.090194 67.274177) (width 0.25) (layer F.Cu) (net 25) (status 20))
 (segment (start 149.098 78.213) (end 148.922999 78.388001) (width 0.25) (layer F.Cu) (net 19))
 (segment (start 145.393138 76.148367) (end 145.393138 75.90088) (width 0.25) (layer F.Cu) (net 19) (status 30))
 (segment (start 148.922999 78.388001) (end 147.632772 78.388001) (width 0.25) (layer F.Cu) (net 19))
 (segment (start 147.632772 78.388001) (end 145.393138 76.148367) (width 0.25) (layer F.Cu) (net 19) (status 20))
 (via (at 149.098 78.213) (size 0.6) (drill 0.4) (layers F.Cu B.Cu) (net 19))
 (segment (start 170.503 70.231) (end 169.3945 71.3395) (width 0.25) (layer B.Cu) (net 19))
 (segment (start 150.020801 78.388001) (end 149.273001 78.388001) (width 0.25) (layer B.Cu) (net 19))
 (segment (start 169.3945 71.3395) (end 157.069302 71.3395) (width 0.25) (layer B.Cu) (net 19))
 (segment (start 171.778 70.231) (end 170.503 70.231) (width 0.25) (layer B.Cu) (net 19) (status 10))
 (segment (start 157.069302 71.3395) (end 150.020801 78.388001) (width 0.25) (layer B.Cu) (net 19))
 (segment (start 149.273001 78.388001) (end 149.098 78.213) (width 0.25) (layer B.Cu) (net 19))
 (segment (start 147.446374 78.837999) (end 145.07494 76.466565) (width 0.25) (layer F.Cu) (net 18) (status 20))
 (segment (start 149.098 79.013) (end 148.922999 78.837999) (width 0.25) (layer F.Cu) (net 18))
 (segment (start 148.922999 78.837999) (end 147.446374 78.837999) (width 0.25) (layer F.Cu) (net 18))
 (segment (start 145.07494 76.466565) (end 144.827452 76.466565) (width 0.25) (layer F.Cu) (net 18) (status 30))
 (via (at 149.098 79.013) (size 0.6) (drill 0.4) (layers F.Cu B.Cu) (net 18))
 (segment (start 149.273001 78.837999) (end 149.098 79.013) (width 0.25) (layer B.Cu) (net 18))
 (segment (start 171.778 72.898) (end 170.503 72.898) (width 0.25) (layer B.Cu) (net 18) (status 10))
 (segment (start 170.503 72.898) (end 169.3945 71.7895) (width 0.25) (layer B.Cu) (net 18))
 (segment (start 169.3945 71.7895) (end 157.255698 71.7895) (width 0.25) (layer B.Cu) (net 18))
 (segment (start 157.255698 71.7895) (end 150.207199 78.837999) (width 0.25) (layer B.Cu) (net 18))
 (segment (start 150.207199 78.837999) (end 149.273001 78.837999) (width 0.25) (layer B.Cu) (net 18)))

